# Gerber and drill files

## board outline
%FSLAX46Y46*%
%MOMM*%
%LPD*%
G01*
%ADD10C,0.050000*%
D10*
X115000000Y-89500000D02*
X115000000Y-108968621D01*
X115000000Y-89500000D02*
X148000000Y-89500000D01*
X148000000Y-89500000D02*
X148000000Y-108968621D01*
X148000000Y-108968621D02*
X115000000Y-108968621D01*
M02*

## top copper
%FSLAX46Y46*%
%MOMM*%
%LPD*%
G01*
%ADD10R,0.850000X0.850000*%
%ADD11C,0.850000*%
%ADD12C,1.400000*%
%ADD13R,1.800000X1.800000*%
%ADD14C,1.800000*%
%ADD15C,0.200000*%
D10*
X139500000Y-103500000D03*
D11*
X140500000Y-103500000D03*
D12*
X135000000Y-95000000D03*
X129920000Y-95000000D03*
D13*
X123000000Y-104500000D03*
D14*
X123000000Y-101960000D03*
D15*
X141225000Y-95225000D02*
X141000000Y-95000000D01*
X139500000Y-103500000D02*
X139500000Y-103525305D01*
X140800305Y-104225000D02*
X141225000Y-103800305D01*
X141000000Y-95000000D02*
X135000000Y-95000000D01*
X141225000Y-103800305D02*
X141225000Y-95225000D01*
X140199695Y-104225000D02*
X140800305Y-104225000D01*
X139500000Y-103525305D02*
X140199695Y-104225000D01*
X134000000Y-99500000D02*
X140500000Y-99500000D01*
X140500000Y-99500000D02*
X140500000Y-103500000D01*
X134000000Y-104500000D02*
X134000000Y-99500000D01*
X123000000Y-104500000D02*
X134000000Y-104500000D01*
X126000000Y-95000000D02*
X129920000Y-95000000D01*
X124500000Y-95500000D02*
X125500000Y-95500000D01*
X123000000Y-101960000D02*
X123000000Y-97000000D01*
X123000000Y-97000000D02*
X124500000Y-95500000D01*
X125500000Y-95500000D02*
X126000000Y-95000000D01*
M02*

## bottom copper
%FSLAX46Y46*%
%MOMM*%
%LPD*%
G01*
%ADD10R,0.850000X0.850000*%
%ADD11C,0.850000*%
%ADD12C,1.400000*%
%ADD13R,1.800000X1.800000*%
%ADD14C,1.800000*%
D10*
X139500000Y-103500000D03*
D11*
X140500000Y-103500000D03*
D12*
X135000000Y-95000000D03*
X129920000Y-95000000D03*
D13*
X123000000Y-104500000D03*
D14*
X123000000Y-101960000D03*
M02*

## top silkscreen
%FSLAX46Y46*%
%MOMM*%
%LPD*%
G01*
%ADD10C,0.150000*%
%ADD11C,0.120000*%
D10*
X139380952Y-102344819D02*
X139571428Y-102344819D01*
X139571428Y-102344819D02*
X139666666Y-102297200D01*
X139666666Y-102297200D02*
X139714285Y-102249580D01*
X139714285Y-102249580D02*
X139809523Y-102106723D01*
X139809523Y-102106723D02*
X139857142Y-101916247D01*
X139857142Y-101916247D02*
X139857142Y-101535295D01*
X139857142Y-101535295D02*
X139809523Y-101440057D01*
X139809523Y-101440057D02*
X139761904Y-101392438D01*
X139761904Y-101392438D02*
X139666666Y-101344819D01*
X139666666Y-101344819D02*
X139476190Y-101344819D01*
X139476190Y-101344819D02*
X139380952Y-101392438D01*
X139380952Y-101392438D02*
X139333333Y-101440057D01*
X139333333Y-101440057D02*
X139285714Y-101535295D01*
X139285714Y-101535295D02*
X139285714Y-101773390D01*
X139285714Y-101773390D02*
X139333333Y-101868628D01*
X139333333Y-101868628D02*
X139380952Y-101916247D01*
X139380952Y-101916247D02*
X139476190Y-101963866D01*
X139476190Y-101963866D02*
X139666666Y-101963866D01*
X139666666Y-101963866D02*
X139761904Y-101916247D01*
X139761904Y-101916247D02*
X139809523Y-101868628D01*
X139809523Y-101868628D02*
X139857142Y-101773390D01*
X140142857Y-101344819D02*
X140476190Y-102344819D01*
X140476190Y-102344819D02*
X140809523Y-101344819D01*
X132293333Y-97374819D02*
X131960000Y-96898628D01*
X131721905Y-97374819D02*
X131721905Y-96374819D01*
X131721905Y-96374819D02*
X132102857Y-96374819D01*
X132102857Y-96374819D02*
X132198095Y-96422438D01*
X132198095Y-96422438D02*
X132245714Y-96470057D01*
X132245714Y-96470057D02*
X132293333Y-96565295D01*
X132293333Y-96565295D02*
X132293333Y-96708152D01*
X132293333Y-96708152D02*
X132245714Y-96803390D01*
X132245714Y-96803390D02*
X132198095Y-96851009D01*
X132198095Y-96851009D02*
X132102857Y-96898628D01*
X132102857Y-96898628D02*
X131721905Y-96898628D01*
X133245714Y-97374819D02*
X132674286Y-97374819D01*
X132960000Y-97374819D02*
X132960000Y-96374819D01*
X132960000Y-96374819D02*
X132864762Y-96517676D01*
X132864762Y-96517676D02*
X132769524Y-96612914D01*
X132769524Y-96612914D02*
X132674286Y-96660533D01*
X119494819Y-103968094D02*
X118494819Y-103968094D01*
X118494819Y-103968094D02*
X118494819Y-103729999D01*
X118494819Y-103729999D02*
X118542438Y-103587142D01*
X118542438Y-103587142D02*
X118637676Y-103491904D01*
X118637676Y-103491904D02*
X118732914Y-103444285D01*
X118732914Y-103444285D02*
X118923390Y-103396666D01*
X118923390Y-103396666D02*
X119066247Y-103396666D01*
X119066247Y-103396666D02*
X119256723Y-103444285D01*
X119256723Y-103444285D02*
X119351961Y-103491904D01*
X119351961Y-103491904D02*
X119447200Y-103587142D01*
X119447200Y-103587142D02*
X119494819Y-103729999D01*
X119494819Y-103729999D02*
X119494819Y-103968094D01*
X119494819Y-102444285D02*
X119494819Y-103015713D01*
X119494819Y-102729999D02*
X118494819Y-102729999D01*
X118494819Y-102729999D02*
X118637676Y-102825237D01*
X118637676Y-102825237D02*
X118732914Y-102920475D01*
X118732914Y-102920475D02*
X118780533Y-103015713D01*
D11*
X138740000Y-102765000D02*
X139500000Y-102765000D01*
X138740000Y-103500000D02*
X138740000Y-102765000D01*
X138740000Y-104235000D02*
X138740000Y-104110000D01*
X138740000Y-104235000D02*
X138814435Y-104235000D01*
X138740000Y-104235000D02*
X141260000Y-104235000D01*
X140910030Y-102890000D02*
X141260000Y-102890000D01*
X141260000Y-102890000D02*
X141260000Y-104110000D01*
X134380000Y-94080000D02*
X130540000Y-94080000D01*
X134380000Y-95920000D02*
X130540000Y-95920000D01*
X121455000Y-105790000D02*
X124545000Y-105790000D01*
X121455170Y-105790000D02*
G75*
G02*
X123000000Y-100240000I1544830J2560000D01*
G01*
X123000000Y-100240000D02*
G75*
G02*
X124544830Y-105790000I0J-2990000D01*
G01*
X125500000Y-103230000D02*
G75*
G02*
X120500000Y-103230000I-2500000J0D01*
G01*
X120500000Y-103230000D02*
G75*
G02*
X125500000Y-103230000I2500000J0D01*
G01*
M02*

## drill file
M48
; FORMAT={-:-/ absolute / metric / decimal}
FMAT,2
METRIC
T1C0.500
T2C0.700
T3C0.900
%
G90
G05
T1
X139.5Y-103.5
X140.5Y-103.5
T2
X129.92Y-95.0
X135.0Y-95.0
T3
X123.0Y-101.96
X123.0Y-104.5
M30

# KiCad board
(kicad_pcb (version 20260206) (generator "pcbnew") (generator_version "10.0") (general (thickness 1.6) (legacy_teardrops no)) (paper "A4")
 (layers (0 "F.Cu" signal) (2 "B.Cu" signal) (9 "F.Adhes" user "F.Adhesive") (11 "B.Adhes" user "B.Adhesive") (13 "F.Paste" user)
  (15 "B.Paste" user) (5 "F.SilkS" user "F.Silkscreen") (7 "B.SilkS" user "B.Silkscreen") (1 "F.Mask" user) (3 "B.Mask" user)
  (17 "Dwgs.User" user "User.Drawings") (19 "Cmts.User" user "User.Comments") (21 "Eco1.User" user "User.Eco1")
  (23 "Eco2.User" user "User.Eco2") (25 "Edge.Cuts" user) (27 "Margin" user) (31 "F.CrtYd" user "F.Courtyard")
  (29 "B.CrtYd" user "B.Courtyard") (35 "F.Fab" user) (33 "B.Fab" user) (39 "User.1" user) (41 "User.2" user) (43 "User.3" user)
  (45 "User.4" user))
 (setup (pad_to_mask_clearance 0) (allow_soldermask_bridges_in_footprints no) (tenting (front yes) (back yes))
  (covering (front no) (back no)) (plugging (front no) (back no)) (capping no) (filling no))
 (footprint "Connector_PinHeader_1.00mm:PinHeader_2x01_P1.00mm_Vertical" (layer "F.Cu") (at 139.5 103.5)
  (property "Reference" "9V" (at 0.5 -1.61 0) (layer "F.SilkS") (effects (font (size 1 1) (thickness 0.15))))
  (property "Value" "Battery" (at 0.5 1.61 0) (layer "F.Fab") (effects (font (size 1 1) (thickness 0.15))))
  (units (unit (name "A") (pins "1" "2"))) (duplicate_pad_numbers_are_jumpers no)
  (fp_line (start -0.76 -0.735) (end 0 -0.735) (stroke (width 0.12) (type solid)) (layer "F.SilkS"))
  (fp_line (start -0.76 0) (end -0.76 -0.735) (stroke (width 0.12) (type solid)) (layer "F.SilkS"))
  (fp_line (start -0.76 0.735) (end -0.76 0.61) (stroke (width 0.12) (type solid)) (layer "F.SilkS"))
  (fp_line (start -0.76 0.735) (end -0.685565 0.735) (stroke (width 0.12) (type solid)) (layer "F.SilkS"))
  (fp_line (start -0.76 0.735) (end 1.76 0.735) (stroke (width 0.12) (type solid)) (layer "F.SilkS"))
  (fp_line (start 1.41003 -0.61) (end 1.76 -0.61) (stroke (width 0.12) (type solid)) (layer "F.SilkS"))
  (fp_line (start 1.76 -0.61) (end 1.76 0.61) (stroke (width 0.12) (type solid)) (layer "F.SilkS"))
  (pad "1" thru_hole rect (at 0 0) (size 0.85 0.85) (drill 0.5) (layers "*.Cu" "*.Mask") (remove_unused_layers no) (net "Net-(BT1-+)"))
  (pad "2" thru_hole circle (at 1 0) (size 0.85 0.85) (drill 0.5) (layers "*.Cu" "*.Mask") (remove_unused_layers no) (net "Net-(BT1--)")))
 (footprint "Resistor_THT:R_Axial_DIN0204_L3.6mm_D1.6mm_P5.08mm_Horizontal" (layer "F.Cu") (at 135 95 180)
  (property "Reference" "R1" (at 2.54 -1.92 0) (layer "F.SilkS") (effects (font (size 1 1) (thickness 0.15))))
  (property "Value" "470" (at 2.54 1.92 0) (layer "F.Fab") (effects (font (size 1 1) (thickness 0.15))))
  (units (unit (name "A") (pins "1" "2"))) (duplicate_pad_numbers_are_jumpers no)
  (fp_line (start 0.62 0.92) (end 4.46 0.92) (stroke (width 0.12) (type solid)) (layer "F.SilkS"))
  (fp_line (start 0.62 -0.92) (end 4.46 -0.92) (stroke (width 0.12) (type solid)) (layer "F.SilkS"))
  (pad "1" thru_hole circle (at 0 0 180) (size 1.4 1.4) (drill 0.7) (layers "*.Cu" "*.Mask") (remove_unused_layers no) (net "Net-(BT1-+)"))
  (pad "2" thru_hole circle (at 5.08 0 180) (size 1.4 1.4) (drill 0.7) (layers "*.Cu" "*.Mask") (remove_unused_layers no) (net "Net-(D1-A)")))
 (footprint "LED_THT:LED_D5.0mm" (layer "F.Cu") (at 123 104.5 90)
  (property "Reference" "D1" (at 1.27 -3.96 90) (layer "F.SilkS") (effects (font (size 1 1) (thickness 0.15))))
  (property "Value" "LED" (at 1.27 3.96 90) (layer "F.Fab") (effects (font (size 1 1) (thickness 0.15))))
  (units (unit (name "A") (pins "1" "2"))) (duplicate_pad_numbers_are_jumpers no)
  (fp_line (start -1.29 -1.545) (end -1.29 1.545) (stroke (width 0.12) (type solid)) (layer "F.SilkS"))
  (fp_arc (start -1.29 -1.54483) (mid 2.071779 -2.880495) (end 4.26 0) (stroke (width 0.12) (type solid)) (layer "F.SilkS"))
  (fp_arc (start 4.26 0) (mid 2.071779 2.880495) (end -1.29 1.54483) (stroke (width 0.12) (type solid)) (layer "F.SilkS"))
  (fp_circle (center 1.27 0) (end 3.77 0) (stroke (width 0.12) (type solid)) (fill no) (layer "F.SilkS"))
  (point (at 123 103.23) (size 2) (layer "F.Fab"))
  (pad "1" thru_hole rect (at 0 0 90) (size 1.8 1.8) (drill 0.9) (layers "*.Cu" "*.Mask") (remove_unused_layers no) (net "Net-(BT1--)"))
  (pad "2" thru_hole circle (at 2.54 0 90) (size 1.8 1.8) (drill 0.9) (layers "*.Cu" "*.Mask") (remove_unused_layers no) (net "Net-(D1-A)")))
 (gr_line (start 115 89.5) (end 115 108.968621) (stroke (width 0.05) (type default)) (layer "Edge.Cuts"))
 (gr_line (start 115 89.5) (end 148 89.5) (stroke (width 0.05) (type default)) (layer "Edge.Cuts"))
 (gr_line (start 148 89.5) (end 148 108.968621) (stroke (width 0.05) (type default)) (layer "Edge.Cuts"))
 (gr_line (start 148 108.968621) (end 115 108.968621) (stroke (width 0.05) (type default)) (layer "Edge.Cuts"))
 (segment (start 141.225 95.225) (end 141 95) (width 0.2) (layer "F.Cu") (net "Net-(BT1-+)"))
 (segment (start 139.5 103.5) (end 139.5 103.525305) (width 0.2) (layer "F.Cu") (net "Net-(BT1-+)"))
 (segment (start 140.800305 104.225) (end 141.225 103.800305) (width 0.2) (layer "F.Cu") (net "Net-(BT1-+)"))
 (segment (start 141 95) (end 135 95) (width 0.2) (layer "F.Cu") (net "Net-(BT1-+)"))
 (segment (start 141.225 103.800305) (end 141.225 95.225) (width 0.2) (layer "F.Cu") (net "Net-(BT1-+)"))
 (segment (start 140.199695 104.225) (end 140.800305 104.225) (width 0.2) (layer "F.Cu") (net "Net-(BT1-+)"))
 (segment (start 139.5 103.525305) (end 140.199695 104.225) (width 0.2) (layer "F.Cu") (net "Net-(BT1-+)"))
 (segment (start 134 99.5) (end 140.5 99.5) (width 0.2) (layer "F.Cu") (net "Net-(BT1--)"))
 (segment (start 140.5 99.5) (end 140.5 103.5) (width 0.2) (layer "F.Cu") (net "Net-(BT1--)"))
 (segment (start 134 104.5) (end 134 99.5) (width 0.2) (layer "F.Cu") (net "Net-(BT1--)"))
 (segment (start 123 104.5) (end 134 104.5) (width 0.2) (layer "F.Cu") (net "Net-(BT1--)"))
 (segment (start 126 95) (end 129.92 95) (width 0.2) (layer "F.Cu") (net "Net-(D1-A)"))
 (segment (start 124.5 95.5) (end 125.5 95.5) (width 0.2) (layer "F.Cu") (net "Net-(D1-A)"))
 (segment (start 123 101.96) (end 123 97) (width 0.2) (layer "F.Cu") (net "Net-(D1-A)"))
 (segment (start 123 97) (end 124.5 95.5) (width 0.2) (layer "F.Cu") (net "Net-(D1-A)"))
 (segment (start 125.5 95.5) (end 126 95) (width 0.2) (layer "F.Cu") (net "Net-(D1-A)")))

